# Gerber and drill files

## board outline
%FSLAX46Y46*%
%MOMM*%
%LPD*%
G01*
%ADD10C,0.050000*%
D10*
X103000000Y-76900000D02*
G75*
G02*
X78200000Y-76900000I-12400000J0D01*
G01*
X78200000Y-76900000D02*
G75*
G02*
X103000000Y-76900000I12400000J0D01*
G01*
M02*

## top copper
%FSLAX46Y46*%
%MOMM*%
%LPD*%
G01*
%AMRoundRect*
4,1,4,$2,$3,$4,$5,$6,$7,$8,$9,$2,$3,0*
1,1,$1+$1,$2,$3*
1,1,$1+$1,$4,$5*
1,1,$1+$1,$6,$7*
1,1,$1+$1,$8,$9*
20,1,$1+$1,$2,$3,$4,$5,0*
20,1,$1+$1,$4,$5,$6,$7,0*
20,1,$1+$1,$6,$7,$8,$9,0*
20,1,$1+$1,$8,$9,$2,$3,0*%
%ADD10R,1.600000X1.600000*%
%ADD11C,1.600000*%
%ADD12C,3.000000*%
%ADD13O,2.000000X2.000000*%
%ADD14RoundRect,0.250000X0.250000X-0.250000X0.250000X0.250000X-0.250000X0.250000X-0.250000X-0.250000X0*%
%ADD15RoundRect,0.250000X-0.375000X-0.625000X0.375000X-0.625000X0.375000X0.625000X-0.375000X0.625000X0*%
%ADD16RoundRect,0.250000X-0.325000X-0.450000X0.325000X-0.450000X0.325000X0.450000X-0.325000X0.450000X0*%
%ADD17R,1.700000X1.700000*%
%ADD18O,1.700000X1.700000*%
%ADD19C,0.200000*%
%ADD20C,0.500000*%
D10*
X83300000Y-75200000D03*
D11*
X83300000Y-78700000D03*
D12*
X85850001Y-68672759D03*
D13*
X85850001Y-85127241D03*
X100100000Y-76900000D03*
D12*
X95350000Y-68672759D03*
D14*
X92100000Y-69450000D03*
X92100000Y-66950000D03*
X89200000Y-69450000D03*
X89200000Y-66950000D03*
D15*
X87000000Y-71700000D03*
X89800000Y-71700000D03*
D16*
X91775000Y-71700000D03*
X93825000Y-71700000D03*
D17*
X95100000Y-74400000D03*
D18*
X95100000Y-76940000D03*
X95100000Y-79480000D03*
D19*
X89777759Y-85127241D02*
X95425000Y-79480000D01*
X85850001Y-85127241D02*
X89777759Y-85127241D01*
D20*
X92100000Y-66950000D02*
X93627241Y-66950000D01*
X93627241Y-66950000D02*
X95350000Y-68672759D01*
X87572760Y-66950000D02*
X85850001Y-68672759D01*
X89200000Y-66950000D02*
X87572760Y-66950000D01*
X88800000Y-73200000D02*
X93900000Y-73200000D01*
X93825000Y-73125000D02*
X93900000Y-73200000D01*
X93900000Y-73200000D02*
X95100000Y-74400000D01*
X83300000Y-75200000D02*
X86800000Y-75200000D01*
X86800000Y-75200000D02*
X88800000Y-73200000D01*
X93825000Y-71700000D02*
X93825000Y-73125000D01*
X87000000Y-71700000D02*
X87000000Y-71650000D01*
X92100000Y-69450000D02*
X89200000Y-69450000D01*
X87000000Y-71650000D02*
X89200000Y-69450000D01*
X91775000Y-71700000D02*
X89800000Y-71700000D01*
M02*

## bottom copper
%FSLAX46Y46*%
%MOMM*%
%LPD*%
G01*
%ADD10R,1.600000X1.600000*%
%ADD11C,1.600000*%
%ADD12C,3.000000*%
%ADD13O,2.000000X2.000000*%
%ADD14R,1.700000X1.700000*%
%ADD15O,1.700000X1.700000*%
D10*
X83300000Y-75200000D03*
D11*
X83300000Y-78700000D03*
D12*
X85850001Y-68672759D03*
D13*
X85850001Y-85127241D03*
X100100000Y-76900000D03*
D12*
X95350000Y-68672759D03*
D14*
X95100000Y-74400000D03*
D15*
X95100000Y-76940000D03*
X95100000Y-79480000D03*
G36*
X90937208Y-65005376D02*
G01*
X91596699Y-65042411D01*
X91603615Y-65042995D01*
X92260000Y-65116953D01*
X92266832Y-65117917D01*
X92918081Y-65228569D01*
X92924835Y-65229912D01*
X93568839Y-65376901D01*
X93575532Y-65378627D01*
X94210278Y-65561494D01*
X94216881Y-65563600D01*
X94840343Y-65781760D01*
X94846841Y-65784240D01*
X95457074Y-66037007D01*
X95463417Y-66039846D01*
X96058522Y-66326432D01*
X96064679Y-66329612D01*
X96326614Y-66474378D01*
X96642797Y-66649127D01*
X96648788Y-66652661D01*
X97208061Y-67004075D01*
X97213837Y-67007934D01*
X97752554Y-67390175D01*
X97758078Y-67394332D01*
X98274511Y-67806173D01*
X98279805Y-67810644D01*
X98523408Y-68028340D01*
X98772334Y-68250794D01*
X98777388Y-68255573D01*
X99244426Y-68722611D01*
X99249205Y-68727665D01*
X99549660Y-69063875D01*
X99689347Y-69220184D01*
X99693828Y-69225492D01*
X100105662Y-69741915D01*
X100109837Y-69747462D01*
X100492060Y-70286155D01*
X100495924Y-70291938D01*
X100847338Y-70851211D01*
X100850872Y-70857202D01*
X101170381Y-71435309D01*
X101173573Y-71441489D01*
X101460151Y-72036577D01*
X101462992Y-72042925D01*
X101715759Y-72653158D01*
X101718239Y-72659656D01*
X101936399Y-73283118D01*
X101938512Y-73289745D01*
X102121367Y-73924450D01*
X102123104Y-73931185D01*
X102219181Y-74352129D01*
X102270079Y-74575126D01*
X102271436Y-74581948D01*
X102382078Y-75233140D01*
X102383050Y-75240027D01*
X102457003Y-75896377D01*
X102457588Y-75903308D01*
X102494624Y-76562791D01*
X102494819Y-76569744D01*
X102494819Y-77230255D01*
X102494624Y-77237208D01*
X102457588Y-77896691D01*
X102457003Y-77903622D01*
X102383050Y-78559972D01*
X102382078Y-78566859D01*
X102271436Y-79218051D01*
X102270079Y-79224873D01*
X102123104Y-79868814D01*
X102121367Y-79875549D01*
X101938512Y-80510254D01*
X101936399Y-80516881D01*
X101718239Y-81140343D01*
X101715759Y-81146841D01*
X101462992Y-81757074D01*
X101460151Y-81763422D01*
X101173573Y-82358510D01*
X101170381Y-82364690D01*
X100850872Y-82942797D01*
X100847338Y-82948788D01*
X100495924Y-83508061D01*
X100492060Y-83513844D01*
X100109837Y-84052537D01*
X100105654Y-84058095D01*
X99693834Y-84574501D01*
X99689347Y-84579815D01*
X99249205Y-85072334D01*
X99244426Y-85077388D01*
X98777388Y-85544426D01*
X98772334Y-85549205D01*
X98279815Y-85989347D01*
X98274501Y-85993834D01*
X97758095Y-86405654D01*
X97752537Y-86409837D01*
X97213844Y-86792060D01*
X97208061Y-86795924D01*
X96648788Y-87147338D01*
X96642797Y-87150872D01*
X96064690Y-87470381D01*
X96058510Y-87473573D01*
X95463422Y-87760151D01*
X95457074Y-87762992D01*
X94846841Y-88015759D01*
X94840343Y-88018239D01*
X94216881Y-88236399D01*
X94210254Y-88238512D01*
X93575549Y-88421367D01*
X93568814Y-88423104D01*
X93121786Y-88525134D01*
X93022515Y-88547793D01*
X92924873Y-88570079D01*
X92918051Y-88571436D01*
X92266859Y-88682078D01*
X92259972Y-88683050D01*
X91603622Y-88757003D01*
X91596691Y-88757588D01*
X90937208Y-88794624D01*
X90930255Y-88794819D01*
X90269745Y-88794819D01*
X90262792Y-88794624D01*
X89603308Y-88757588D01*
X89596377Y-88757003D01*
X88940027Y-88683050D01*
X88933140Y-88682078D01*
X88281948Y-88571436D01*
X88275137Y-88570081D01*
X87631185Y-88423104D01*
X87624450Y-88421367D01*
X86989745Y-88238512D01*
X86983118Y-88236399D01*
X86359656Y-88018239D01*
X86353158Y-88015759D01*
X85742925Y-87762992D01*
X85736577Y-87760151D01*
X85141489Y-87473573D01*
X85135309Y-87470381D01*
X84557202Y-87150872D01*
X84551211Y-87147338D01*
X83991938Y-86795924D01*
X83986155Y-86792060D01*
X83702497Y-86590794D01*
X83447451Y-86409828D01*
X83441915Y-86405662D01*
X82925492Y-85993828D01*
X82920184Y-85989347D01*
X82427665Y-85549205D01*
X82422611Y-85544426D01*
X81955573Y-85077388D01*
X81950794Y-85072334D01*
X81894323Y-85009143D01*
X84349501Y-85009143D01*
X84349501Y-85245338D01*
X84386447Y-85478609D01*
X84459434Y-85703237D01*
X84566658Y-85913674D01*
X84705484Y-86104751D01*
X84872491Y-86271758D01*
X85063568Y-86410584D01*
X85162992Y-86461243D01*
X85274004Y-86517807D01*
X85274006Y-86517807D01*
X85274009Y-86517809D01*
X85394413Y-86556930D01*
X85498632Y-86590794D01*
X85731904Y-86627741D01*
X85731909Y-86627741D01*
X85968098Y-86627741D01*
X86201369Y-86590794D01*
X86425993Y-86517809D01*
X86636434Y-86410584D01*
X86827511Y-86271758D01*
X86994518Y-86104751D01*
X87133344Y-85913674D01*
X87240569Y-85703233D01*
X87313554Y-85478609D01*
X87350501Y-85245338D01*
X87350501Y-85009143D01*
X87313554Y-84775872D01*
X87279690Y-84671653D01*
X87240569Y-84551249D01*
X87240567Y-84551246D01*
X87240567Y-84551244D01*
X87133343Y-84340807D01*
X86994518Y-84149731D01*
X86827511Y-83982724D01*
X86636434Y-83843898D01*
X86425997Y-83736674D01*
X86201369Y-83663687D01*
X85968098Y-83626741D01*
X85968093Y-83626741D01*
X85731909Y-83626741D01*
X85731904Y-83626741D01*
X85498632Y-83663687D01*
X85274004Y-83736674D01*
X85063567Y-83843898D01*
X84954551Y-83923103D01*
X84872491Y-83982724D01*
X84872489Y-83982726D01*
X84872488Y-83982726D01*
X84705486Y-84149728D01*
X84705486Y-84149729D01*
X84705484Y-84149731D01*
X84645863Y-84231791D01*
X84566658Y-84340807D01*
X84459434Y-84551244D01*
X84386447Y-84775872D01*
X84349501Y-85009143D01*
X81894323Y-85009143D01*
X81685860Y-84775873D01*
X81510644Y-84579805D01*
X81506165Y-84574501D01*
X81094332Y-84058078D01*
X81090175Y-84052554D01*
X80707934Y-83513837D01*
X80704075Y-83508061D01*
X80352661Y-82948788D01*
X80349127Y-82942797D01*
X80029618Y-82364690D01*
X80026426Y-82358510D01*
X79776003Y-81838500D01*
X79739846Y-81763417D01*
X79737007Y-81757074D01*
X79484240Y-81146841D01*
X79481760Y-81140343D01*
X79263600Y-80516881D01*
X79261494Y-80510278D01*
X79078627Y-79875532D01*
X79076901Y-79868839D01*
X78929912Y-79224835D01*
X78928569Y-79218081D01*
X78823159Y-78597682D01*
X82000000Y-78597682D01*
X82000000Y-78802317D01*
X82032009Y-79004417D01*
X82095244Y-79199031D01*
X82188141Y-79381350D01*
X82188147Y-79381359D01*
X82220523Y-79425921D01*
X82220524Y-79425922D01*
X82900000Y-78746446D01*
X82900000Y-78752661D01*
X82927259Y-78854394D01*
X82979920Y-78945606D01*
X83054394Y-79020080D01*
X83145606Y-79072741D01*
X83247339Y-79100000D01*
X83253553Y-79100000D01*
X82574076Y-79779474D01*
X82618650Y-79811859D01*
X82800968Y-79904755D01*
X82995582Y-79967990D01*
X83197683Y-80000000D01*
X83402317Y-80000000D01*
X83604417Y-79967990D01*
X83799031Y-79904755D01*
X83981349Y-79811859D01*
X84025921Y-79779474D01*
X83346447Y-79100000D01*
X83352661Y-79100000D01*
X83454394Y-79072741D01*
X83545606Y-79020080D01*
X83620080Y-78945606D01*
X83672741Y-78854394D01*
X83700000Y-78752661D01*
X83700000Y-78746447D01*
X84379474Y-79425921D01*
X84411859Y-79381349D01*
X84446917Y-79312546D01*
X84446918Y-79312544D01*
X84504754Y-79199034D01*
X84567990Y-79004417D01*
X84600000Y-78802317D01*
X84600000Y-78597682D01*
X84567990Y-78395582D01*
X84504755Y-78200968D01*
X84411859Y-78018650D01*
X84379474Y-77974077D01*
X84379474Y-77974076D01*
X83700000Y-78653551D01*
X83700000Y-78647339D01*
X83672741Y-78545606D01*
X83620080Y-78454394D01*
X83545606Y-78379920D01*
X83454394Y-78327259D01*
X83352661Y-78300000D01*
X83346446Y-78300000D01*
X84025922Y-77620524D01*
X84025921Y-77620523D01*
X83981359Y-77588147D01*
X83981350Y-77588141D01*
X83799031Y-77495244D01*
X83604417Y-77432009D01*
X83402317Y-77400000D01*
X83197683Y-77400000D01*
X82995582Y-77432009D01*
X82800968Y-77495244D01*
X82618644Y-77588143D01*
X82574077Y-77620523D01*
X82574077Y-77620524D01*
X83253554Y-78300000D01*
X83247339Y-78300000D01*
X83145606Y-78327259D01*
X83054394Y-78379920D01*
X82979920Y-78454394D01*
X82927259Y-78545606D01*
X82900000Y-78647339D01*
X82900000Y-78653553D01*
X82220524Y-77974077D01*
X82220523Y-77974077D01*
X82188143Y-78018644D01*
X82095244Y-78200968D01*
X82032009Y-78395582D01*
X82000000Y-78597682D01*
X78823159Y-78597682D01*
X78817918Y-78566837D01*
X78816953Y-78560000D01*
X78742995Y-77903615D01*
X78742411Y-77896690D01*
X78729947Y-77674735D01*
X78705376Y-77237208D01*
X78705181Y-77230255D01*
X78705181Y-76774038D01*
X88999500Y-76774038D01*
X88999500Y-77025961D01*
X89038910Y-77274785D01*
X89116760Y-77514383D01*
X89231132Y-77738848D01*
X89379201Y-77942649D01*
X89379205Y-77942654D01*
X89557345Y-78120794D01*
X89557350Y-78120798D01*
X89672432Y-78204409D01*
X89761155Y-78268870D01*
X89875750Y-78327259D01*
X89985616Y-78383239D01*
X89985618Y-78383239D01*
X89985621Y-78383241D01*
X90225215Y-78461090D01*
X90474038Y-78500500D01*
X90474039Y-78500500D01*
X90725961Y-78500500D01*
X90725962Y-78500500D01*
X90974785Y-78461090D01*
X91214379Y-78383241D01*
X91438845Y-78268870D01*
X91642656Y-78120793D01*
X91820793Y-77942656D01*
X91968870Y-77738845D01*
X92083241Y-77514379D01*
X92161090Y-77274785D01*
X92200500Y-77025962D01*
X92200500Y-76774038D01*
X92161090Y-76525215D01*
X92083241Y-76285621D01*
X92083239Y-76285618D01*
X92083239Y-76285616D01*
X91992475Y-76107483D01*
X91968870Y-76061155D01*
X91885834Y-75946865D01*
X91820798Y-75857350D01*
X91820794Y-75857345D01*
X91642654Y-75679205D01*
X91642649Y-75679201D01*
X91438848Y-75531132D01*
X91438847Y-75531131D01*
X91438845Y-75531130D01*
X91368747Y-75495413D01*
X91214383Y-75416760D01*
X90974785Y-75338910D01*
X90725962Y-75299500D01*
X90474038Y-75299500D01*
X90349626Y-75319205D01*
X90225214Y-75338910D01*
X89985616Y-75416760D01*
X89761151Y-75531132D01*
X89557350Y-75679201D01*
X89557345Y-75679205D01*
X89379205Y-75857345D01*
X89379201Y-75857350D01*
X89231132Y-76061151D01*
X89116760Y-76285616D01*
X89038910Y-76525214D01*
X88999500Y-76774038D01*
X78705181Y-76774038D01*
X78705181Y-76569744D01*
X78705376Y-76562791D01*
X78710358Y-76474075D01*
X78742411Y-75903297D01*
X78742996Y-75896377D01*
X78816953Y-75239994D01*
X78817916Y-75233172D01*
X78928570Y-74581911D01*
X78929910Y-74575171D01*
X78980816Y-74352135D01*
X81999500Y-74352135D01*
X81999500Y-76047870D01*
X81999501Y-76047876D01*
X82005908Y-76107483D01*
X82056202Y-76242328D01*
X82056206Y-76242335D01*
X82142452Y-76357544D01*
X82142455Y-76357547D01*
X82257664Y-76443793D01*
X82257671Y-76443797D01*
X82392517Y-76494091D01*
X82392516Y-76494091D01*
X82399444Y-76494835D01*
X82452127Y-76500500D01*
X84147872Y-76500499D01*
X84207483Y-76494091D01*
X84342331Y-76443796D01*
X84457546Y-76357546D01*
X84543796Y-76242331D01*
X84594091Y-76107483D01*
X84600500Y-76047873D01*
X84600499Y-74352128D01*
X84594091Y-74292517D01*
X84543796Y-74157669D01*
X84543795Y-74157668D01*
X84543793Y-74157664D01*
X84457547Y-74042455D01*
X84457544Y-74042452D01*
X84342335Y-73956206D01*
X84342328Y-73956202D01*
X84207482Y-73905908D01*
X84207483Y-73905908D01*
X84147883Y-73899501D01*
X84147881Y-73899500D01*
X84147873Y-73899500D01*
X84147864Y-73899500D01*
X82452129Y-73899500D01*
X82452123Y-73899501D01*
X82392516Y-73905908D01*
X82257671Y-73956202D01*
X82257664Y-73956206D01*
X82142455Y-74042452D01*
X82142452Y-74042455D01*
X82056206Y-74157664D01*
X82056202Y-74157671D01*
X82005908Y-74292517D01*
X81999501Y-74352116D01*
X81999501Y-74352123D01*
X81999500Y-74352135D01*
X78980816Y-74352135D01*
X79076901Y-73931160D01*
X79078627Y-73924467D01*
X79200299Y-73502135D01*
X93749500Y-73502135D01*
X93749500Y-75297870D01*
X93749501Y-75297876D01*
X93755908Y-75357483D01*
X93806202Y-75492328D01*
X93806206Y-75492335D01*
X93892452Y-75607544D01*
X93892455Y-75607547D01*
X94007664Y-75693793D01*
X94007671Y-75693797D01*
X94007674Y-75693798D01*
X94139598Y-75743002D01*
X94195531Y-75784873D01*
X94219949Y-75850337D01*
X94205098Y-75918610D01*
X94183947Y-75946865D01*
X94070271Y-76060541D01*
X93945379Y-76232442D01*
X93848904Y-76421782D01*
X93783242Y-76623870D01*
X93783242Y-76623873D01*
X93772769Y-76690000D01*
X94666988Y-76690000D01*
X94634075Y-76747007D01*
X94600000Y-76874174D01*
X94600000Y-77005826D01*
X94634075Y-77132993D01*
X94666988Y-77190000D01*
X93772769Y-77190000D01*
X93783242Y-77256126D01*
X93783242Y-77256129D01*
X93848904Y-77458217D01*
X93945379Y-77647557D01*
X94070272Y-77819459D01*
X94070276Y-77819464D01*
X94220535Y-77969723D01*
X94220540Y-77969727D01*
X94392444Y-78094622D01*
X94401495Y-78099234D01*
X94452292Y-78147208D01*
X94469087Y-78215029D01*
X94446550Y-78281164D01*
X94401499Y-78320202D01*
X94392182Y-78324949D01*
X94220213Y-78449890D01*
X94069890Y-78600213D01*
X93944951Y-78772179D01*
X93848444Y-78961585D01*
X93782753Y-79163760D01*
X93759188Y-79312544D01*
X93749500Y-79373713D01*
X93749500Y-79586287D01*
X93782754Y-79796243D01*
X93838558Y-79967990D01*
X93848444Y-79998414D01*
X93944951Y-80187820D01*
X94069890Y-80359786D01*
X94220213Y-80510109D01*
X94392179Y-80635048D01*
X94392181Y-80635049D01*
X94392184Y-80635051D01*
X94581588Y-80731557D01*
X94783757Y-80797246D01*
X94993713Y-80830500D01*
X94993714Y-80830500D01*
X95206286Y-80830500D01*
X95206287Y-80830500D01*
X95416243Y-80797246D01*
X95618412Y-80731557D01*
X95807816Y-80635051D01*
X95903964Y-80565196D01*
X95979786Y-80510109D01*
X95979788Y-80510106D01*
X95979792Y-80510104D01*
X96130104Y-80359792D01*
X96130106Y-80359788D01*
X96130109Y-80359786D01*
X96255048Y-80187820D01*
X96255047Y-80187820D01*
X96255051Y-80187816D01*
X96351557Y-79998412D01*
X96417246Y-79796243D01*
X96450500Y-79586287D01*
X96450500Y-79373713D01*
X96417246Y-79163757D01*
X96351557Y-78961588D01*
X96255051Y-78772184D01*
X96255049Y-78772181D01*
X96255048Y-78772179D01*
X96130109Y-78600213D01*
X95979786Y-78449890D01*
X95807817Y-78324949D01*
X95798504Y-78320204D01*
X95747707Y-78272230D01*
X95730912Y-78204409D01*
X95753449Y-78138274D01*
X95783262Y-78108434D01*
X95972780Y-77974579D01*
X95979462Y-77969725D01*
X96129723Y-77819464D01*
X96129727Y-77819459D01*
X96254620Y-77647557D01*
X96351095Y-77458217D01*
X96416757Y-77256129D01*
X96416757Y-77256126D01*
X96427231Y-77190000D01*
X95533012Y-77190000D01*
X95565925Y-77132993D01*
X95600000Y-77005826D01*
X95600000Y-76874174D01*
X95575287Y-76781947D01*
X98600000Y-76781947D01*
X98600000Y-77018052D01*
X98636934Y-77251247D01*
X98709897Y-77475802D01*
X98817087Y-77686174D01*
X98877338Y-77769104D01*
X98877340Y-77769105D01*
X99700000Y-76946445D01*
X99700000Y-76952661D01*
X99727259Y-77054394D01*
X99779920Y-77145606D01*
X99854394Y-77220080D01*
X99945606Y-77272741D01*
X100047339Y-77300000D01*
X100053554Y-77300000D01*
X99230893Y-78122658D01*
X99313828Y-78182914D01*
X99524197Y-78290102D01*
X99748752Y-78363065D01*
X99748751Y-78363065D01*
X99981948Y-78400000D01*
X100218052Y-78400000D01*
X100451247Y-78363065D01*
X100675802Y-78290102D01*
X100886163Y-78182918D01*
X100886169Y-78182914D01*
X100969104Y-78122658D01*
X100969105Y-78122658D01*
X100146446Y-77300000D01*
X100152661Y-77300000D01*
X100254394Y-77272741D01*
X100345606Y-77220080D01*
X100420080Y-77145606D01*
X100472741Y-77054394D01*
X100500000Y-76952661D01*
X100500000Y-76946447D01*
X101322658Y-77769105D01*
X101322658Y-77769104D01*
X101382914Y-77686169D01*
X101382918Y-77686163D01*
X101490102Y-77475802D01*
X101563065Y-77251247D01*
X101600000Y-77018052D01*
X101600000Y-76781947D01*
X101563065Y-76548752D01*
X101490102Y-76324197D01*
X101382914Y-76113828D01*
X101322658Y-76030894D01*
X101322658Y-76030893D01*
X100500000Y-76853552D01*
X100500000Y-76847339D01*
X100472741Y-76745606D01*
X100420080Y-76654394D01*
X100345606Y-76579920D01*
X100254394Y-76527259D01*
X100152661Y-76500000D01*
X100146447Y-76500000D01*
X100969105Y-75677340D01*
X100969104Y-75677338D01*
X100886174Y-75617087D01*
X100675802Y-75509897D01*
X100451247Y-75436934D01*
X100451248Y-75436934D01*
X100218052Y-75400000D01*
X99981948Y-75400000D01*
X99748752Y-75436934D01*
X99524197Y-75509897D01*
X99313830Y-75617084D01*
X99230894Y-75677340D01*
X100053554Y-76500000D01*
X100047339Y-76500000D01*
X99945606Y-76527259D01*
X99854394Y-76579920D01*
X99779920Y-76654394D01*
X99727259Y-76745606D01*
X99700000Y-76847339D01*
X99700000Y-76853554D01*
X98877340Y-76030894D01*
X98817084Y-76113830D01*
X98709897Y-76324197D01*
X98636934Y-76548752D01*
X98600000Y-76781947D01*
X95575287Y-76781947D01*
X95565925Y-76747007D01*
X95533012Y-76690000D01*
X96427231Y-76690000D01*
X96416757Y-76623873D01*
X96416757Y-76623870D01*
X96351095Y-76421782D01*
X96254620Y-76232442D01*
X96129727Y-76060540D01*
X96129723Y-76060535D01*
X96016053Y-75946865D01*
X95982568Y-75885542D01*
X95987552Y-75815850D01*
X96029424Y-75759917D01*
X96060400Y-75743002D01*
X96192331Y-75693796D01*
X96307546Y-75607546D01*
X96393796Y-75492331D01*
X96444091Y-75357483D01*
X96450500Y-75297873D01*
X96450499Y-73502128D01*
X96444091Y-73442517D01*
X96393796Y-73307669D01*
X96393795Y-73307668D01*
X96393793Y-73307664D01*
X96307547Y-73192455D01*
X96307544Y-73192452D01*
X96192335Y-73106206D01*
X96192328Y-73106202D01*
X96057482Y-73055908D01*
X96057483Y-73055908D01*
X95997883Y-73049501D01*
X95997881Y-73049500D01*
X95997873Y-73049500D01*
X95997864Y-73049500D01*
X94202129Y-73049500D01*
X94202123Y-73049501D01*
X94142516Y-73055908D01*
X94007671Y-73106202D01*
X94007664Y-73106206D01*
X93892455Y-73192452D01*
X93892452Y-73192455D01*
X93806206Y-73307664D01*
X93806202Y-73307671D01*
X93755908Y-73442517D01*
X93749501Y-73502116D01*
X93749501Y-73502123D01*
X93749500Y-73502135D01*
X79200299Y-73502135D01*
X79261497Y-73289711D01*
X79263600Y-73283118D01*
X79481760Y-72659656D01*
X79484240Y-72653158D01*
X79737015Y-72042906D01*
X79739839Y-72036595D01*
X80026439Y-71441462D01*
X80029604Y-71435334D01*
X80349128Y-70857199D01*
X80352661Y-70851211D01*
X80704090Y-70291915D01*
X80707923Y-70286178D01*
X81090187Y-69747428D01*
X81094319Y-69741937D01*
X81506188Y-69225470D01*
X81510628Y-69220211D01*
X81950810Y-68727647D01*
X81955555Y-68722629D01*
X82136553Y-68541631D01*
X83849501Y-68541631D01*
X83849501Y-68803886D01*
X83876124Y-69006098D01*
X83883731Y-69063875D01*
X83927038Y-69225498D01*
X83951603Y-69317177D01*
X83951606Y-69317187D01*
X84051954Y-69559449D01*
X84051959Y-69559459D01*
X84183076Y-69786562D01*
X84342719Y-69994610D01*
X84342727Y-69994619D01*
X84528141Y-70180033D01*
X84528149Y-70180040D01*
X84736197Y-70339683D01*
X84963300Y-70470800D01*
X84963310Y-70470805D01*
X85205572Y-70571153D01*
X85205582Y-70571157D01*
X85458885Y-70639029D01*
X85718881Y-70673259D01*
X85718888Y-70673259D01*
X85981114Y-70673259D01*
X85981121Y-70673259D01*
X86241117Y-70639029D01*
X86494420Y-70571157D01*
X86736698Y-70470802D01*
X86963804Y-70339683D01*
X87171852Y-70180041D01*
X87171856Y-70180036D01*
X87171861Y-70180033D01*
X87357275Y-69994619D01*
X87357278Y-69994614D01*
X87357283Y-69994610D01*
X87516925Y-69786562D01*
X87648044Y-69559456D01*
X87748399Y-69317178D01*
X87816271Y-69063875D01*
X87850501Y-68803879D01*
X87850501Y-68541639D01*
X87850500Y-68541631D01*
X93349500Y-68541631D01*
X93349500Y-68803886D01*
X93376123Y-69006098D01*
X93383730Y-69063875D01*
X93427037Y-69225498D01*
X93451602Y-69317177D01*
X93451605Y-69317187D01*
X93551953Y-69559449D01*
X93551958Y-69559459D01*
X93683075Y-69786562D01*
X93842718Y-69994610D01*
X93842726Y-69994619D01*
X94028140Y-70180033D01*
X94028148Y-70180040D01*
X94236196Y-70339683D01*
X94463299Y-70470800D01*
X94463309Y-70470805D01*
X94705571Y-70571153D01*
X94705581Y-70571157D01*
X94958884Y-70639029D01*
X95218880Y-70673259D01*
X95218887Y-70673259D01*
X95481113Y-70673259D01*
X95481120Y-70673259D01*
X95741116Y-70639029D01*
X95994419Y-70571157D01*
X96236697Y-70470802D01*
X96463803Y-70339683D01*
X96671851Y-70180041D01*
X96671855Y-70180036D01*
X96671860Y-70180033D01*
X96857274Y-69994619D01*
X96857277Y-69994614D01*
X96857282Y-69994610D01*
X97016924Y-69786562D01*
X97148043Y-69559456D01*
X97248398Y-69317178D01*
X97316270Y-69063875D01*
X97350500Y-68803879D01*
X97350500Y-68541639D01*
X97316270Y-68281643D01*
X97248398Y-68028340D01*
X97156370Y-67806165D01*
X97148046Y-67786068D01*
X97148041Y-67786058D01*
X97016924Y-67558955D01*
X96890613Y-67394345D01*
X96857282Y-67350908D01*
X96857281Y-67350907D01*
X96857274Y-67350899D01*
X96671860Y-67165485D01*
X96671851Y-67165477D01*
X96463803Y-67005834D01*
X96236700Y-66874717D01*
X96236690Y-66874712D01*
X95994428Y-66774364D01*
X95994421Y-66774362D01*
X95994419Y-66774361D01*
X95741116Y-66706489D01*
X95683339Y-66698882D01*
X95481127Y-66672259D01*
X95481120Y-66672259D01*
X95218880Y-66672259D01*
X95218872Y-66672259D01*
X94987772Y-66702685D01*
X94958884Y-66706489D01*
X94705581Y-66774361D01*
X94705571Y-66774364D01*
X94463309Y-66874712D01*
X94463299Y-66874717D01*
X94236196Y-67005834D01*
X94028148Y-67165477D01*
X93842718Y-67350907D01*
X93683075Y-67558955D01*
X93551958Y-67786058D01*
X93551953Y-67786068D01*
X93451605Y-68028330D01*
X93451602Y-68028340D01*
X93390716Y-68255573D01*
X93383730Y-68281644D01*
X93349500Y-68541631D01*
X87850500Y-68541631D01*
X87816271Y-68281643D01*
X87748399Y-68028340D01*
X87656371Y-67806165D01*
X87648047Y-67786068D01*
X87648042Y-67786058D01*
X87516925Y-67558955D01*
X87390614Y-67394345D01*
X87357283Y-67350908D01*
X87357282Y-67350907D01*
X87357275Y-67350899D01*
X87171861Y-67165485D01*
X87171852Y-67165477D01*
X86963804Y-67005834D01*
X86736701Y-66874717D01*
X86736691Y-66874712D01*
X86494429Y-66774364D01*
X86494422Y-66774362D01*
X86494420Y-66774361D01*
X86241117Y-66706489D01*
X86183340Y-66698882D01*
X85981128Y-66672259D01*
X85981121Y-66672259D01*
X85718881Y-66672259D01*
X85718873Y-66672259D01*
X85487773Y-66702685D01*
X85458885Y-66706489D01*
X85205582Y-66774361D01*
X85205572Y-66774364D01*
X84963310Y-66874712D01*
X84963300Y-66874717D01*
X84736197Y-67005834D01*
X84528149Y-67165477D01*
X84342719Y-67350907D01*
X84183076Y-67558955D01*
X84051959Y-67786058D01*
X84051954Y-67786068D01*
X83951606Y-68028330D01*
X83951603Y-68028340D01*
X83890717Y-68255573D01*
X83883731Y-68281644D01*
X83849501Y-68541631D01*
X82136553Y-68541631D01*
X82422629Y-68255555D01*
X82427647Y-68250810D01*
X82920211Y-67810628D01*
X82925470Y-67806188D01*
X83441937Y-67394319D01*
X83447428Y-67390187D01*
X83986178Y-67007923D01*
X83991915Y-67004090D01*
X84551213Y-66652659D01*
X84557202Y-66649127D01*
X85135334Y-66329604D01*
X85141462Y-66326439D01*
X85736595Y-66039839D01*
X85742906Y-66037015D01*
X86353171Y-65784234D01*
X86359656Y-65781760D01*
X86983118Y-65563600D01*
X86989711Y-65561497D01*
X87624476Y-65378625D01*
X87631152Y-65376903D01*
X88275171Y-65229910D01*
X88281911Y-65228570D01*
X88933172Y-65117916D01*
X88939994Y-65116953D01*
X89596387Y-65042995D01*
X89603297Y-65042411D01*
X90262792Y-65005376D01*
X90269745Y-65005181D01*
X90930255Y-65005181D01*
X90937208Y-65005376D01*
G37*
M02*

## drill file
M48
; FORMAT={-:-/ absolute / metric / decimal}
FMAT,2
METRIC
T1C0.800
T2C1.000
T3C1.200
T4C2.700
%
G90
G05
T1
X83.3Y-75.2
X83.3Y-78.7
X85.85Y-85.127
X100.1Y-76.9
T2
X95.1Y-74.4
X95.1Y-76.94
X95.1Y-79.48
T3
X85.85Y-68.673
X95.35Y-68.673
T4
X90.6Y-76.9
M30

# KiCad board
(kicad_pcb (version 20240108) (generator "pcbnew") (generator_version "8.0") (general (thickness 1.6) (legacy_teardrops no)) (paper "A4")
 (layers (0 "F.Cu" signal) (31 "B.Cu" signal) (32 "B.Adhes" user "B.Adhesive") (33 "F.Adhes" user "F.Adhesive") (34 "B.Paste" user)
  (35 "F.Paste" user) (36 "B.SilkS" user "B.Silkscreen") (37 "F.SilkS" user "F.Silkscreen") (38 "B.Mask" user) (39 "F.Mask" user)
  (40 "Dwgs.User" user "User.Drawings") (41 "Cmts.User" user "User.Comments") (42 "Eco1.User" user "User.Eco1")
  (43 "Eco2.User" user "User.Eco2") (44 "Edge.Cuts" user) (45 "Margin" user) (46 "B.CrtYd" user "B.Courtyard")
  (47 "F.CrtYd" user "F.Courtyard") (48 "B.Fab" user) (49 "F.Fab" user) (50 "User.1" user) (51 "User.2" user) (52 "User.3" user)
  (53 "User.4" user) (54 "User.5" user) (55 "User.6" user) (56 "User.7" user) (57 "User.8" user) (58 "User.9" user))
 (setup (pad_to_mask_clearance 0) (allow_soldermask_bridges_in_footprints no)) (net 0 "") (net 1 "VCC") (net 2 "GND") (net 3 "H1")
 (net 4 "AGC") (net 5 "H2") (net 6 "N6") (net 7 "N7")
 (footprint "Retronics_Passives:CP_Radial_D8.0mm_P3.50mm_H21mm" (layer "F.Cu") (at 83.3 75.2 -90)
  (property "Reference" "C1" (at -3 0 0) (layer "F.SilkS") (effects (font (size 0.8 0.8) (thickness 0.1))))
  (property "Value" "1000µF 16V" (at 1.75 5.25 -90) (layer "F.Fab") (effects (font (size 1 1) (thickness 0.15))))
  (pad "1" thru_hole rect (at 0 0 270) (size 1.6 1.6) (drill 0.8) (layers "*.Cu" "*.Mask") (remove_unused_layers no) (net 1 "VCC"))
  (pad "2" thru_hole circle (at 3.5 0 270) (size 1.6 1.6) (drill 0.8) (layers "*.Cu" "*.Mask") (remove_unused_layers no) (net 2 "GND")))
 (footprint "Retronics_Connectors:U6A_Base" (layer "F.Cu") (at 90.6 76.9)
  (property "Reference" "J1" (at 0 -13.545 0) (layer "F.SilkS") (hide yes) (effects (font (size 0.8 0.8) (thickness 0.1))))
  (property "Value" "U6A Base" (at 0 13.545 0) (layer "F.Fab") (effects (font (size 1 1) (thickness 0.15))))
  (pad "1" thru_hole circle (at -4.749999 -8.227241) (size 3 3) (drill 1.2) (layers "*.Cu" "*.Mask") (remove_unused_layers no) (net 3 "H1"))
  (pad "3" thru_hole oval (at -4.749999 8.227241) (size 2 2) (drill 0.8) (layers "*.Cu" "*.Mask") (remove_unused_layers no) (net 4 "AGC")
   (thermal_bridge_angle 45))
  (pad "5" thru_hole oval (at 9.5 0) (size 2 2) (drill 0.8) (layers "*.Cu" "*.Mask") (remove_unused_layers no) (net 2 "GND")
   (thermal_bridge_angle 45))
  (pad "6" thru_hole circle (at 4.75 -8.227241) (size 3 3) (drill 1.2) (layers "*.Cu" "*.Mask") (remove_unused_layers no) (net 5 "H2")))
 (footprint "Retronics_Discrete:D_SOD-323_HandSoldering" (layer "F.Cu") (at 92.1 68.2 90)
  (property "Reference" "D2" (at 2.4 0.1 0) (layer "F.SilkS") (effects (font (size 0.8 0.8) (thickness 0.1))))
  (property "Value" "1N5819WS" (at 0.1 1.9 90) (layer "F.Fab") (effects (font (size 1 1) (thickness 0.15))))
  (pad "1" smd roundrect (at -1.25 0 90) (size 1 1) (layers "F.Cu" "F.Paste" "F.Mask") (roundrect_rratio 0.25) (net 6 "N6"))
  (pad "2" smd roundrect (at 1.25 0 90) (size 1 1) (layers "F.Cu" "F.Paste" "F.Mask") (roundrect_rratio 0.25) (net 5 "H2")))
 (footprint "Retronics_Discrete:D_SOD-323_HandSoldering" (layer "F.Cu") (at 89.2 68.2 90)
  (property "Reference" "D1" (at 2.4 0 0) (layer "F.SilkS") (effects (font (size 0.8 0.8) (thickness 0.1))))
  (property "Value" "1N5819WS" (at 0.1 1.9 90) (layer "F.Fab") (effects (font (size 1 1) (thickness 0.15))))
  (pad "1" smd roundrect (at -1.25 0 90) (size 1 1) (layers "F.Cu" "F.Paste" "F.Mask") (roundrect_rratio 0.25) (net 6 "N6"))
  (pad "2" smd roundrect (at 1.25 0 90) (size 1 1) (layers "F.Cu" "F.Paste" "F.Mask") (roundrect_rratio 0.25) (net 3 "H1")))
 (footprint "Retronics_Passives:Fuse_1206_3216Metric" (layer "F.Cu") (at 88.4 71.7)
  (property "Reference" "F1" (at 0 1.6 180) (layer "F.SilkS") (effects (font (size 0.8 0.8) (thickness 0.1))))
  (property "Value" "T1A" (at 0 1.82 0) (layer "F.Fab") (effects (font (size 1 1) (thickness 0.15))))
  (pad "1" smd roundrect (at -1.4 0) (size 1.25 1.75) (layers "F.Cu" "F.Paste" "F.Mask") (roundrect_rratio 0.2) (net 6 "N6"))
  (pad "2" smd roundrect (at 1.4 0) (size 1.25 1.75) (layers "F.Cu" "F.Paste" "F.Mask") (roundrect_rratio 0.2) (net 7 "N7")))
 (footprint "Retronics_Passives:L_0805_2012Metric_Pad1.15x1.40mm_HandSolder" (layer "F.Cu") (at 92.8 71.7)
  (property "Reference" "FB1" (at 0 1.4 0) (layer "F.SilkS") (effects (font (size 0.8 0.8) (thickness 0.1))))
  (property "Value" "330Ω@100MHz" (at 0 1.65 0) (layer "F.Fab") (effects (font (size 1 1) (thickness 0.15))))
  (pad "1" smd roundrect (at -1.025 0) (size 1.15 1.4) (layers "F.Cu" "F.Paste" "F.Mask") (roundrect_rratio 0.217391) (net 7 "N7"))
  (pad "2" smd roundrect (at 1.025 0) (size 1.15 1.4) (layers "F.Cu" "F.Paste" "F.Mask") (roundrect_rratio 0.217391) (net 1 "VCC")))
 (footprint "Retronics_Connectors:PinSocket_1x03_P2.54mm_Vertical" (layer "F.Cu") (at 95.1 74.4)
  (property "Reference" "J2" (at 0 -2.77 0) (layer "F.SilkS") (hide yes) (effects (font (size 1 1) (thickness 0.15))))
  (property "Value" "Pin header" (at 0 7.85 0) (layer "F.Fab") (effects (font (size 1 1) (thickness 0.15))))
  (pad "1" thru_hole rect (at 0 0) (size 1.7 1.7) (drill 1) (layers "*.Cu" "*.Mask") (remove_unused_layers no) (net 1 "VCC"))
  (pad "2" thru_hole oval (at 0 2.54) (size 1.7 1.7) (drill 1) (layers "*.Cu" "*.Mask") (remove_unused_layers no) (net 2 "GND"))
  (pad "3" thru_hole oval (at 0 5.08) (size 1.7 1.7) (drill 1) (layers "*.Cu" "*.Mask") (remove_unused_layers no) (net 4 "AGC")))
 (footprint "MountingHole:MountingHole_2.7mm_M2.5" (layer "F.Cu") (at 90.6 76.9)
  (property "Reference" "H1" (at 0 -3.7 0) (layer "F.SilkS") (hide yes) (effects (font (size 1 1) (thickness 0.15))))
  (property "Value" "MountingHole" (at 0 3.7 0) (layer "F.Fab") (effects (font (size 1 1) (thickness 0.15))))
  (pad "" np_thru_hole circle (at 0 0) (size 2.7 2.7) (drill 2.7) (layers "*.Cu" "*.Mask")))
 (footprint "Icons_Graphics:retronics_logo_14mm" (layer "B.Cu") (at 91.7 82.2 180)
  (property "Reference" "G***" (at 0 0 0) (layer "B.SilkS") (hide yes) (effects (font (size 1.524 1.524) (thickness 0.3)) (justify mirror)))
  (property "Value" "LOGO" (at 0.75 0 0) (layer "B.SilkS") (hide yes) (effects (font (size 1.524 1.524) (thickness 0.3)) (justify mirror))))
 (gr_circle (center 90.6 76.9) (end 103 76.9) (stroke (width 0.05) (type default)) (fill none) (layer "Edge.Cuts"))
 (segment (start 89.777759 85.127241) (end 95.425 79.48) (width 0.2) (layer "F.Cu") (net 4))
 (segment (start 85.850001 85.127241) (end 89.777759 85.127241) (width 0.2) (layer "F.Cu") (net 4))
 (segment (start 92.1 66.95) (end 93.627241 66.95) (width 0.5) (layer "F.Cu") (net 5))
 (segment (start 93.627241 66.95) (end 95.35 68.672759) (width 0.5) (layer "F.Cu") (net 5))
 (segment (start 87.57276 66.95) (end 85.850001 68.672759) (width 0.5) (layer "F.Cu") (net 3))
 (segment (start 89.2 66.95) (end 87.57276 66.95) (width 0.5) (layer "F.Cu") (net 3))
 (segment (start 88.8 73.2) (end 93.9 73.2) (width 0.5) (layer "F.Cu") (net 1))
 (segment (start 93.825 73.125) (end 93.9 73.2) (width 0.5) (layer "F.Cu") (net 1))
 (segment (start 93.9 73.2) (end 95.1 74.4) (width 0.5) (layer "F.Cu") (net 1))
 (segment (start 83.3 75.2) (end 86.8 75.2) (width 0.5) (layer "F.Cu") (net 1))
 (segment (start 86.8 75.2) (end 88.8 73.2) (width 0.5) (layer "F.Cu") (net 1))
 (segment (start 93.825 71.7) (end 93.825 73.125) (width 0.5) (layer "F.Cu") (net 1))
 (segment (start 87 71.7) (end 87 71.65) (width 0.5) (layer "F.Cu") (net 6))
 (segment (start 92.1 69.45) (end 89.2 69.45) (width 0.5) (layer "F.Cu") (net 6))
 (segment (start 87 71.65) (end 89.2 69.45) (width 0.5) (layer "F.Cu") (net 6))
 (segment (start 91.775 71.7) (end 89.8 71.7) (width 0.5) (layer "F.Cu") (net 7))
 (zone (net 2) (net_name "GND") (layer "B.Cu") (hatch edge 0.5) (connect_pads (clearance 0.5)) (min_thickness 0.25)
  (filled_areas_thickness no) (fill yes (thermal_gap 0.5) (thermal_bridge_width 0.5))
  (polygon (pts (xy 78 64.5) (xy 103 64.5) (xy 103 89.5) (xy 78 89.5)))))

